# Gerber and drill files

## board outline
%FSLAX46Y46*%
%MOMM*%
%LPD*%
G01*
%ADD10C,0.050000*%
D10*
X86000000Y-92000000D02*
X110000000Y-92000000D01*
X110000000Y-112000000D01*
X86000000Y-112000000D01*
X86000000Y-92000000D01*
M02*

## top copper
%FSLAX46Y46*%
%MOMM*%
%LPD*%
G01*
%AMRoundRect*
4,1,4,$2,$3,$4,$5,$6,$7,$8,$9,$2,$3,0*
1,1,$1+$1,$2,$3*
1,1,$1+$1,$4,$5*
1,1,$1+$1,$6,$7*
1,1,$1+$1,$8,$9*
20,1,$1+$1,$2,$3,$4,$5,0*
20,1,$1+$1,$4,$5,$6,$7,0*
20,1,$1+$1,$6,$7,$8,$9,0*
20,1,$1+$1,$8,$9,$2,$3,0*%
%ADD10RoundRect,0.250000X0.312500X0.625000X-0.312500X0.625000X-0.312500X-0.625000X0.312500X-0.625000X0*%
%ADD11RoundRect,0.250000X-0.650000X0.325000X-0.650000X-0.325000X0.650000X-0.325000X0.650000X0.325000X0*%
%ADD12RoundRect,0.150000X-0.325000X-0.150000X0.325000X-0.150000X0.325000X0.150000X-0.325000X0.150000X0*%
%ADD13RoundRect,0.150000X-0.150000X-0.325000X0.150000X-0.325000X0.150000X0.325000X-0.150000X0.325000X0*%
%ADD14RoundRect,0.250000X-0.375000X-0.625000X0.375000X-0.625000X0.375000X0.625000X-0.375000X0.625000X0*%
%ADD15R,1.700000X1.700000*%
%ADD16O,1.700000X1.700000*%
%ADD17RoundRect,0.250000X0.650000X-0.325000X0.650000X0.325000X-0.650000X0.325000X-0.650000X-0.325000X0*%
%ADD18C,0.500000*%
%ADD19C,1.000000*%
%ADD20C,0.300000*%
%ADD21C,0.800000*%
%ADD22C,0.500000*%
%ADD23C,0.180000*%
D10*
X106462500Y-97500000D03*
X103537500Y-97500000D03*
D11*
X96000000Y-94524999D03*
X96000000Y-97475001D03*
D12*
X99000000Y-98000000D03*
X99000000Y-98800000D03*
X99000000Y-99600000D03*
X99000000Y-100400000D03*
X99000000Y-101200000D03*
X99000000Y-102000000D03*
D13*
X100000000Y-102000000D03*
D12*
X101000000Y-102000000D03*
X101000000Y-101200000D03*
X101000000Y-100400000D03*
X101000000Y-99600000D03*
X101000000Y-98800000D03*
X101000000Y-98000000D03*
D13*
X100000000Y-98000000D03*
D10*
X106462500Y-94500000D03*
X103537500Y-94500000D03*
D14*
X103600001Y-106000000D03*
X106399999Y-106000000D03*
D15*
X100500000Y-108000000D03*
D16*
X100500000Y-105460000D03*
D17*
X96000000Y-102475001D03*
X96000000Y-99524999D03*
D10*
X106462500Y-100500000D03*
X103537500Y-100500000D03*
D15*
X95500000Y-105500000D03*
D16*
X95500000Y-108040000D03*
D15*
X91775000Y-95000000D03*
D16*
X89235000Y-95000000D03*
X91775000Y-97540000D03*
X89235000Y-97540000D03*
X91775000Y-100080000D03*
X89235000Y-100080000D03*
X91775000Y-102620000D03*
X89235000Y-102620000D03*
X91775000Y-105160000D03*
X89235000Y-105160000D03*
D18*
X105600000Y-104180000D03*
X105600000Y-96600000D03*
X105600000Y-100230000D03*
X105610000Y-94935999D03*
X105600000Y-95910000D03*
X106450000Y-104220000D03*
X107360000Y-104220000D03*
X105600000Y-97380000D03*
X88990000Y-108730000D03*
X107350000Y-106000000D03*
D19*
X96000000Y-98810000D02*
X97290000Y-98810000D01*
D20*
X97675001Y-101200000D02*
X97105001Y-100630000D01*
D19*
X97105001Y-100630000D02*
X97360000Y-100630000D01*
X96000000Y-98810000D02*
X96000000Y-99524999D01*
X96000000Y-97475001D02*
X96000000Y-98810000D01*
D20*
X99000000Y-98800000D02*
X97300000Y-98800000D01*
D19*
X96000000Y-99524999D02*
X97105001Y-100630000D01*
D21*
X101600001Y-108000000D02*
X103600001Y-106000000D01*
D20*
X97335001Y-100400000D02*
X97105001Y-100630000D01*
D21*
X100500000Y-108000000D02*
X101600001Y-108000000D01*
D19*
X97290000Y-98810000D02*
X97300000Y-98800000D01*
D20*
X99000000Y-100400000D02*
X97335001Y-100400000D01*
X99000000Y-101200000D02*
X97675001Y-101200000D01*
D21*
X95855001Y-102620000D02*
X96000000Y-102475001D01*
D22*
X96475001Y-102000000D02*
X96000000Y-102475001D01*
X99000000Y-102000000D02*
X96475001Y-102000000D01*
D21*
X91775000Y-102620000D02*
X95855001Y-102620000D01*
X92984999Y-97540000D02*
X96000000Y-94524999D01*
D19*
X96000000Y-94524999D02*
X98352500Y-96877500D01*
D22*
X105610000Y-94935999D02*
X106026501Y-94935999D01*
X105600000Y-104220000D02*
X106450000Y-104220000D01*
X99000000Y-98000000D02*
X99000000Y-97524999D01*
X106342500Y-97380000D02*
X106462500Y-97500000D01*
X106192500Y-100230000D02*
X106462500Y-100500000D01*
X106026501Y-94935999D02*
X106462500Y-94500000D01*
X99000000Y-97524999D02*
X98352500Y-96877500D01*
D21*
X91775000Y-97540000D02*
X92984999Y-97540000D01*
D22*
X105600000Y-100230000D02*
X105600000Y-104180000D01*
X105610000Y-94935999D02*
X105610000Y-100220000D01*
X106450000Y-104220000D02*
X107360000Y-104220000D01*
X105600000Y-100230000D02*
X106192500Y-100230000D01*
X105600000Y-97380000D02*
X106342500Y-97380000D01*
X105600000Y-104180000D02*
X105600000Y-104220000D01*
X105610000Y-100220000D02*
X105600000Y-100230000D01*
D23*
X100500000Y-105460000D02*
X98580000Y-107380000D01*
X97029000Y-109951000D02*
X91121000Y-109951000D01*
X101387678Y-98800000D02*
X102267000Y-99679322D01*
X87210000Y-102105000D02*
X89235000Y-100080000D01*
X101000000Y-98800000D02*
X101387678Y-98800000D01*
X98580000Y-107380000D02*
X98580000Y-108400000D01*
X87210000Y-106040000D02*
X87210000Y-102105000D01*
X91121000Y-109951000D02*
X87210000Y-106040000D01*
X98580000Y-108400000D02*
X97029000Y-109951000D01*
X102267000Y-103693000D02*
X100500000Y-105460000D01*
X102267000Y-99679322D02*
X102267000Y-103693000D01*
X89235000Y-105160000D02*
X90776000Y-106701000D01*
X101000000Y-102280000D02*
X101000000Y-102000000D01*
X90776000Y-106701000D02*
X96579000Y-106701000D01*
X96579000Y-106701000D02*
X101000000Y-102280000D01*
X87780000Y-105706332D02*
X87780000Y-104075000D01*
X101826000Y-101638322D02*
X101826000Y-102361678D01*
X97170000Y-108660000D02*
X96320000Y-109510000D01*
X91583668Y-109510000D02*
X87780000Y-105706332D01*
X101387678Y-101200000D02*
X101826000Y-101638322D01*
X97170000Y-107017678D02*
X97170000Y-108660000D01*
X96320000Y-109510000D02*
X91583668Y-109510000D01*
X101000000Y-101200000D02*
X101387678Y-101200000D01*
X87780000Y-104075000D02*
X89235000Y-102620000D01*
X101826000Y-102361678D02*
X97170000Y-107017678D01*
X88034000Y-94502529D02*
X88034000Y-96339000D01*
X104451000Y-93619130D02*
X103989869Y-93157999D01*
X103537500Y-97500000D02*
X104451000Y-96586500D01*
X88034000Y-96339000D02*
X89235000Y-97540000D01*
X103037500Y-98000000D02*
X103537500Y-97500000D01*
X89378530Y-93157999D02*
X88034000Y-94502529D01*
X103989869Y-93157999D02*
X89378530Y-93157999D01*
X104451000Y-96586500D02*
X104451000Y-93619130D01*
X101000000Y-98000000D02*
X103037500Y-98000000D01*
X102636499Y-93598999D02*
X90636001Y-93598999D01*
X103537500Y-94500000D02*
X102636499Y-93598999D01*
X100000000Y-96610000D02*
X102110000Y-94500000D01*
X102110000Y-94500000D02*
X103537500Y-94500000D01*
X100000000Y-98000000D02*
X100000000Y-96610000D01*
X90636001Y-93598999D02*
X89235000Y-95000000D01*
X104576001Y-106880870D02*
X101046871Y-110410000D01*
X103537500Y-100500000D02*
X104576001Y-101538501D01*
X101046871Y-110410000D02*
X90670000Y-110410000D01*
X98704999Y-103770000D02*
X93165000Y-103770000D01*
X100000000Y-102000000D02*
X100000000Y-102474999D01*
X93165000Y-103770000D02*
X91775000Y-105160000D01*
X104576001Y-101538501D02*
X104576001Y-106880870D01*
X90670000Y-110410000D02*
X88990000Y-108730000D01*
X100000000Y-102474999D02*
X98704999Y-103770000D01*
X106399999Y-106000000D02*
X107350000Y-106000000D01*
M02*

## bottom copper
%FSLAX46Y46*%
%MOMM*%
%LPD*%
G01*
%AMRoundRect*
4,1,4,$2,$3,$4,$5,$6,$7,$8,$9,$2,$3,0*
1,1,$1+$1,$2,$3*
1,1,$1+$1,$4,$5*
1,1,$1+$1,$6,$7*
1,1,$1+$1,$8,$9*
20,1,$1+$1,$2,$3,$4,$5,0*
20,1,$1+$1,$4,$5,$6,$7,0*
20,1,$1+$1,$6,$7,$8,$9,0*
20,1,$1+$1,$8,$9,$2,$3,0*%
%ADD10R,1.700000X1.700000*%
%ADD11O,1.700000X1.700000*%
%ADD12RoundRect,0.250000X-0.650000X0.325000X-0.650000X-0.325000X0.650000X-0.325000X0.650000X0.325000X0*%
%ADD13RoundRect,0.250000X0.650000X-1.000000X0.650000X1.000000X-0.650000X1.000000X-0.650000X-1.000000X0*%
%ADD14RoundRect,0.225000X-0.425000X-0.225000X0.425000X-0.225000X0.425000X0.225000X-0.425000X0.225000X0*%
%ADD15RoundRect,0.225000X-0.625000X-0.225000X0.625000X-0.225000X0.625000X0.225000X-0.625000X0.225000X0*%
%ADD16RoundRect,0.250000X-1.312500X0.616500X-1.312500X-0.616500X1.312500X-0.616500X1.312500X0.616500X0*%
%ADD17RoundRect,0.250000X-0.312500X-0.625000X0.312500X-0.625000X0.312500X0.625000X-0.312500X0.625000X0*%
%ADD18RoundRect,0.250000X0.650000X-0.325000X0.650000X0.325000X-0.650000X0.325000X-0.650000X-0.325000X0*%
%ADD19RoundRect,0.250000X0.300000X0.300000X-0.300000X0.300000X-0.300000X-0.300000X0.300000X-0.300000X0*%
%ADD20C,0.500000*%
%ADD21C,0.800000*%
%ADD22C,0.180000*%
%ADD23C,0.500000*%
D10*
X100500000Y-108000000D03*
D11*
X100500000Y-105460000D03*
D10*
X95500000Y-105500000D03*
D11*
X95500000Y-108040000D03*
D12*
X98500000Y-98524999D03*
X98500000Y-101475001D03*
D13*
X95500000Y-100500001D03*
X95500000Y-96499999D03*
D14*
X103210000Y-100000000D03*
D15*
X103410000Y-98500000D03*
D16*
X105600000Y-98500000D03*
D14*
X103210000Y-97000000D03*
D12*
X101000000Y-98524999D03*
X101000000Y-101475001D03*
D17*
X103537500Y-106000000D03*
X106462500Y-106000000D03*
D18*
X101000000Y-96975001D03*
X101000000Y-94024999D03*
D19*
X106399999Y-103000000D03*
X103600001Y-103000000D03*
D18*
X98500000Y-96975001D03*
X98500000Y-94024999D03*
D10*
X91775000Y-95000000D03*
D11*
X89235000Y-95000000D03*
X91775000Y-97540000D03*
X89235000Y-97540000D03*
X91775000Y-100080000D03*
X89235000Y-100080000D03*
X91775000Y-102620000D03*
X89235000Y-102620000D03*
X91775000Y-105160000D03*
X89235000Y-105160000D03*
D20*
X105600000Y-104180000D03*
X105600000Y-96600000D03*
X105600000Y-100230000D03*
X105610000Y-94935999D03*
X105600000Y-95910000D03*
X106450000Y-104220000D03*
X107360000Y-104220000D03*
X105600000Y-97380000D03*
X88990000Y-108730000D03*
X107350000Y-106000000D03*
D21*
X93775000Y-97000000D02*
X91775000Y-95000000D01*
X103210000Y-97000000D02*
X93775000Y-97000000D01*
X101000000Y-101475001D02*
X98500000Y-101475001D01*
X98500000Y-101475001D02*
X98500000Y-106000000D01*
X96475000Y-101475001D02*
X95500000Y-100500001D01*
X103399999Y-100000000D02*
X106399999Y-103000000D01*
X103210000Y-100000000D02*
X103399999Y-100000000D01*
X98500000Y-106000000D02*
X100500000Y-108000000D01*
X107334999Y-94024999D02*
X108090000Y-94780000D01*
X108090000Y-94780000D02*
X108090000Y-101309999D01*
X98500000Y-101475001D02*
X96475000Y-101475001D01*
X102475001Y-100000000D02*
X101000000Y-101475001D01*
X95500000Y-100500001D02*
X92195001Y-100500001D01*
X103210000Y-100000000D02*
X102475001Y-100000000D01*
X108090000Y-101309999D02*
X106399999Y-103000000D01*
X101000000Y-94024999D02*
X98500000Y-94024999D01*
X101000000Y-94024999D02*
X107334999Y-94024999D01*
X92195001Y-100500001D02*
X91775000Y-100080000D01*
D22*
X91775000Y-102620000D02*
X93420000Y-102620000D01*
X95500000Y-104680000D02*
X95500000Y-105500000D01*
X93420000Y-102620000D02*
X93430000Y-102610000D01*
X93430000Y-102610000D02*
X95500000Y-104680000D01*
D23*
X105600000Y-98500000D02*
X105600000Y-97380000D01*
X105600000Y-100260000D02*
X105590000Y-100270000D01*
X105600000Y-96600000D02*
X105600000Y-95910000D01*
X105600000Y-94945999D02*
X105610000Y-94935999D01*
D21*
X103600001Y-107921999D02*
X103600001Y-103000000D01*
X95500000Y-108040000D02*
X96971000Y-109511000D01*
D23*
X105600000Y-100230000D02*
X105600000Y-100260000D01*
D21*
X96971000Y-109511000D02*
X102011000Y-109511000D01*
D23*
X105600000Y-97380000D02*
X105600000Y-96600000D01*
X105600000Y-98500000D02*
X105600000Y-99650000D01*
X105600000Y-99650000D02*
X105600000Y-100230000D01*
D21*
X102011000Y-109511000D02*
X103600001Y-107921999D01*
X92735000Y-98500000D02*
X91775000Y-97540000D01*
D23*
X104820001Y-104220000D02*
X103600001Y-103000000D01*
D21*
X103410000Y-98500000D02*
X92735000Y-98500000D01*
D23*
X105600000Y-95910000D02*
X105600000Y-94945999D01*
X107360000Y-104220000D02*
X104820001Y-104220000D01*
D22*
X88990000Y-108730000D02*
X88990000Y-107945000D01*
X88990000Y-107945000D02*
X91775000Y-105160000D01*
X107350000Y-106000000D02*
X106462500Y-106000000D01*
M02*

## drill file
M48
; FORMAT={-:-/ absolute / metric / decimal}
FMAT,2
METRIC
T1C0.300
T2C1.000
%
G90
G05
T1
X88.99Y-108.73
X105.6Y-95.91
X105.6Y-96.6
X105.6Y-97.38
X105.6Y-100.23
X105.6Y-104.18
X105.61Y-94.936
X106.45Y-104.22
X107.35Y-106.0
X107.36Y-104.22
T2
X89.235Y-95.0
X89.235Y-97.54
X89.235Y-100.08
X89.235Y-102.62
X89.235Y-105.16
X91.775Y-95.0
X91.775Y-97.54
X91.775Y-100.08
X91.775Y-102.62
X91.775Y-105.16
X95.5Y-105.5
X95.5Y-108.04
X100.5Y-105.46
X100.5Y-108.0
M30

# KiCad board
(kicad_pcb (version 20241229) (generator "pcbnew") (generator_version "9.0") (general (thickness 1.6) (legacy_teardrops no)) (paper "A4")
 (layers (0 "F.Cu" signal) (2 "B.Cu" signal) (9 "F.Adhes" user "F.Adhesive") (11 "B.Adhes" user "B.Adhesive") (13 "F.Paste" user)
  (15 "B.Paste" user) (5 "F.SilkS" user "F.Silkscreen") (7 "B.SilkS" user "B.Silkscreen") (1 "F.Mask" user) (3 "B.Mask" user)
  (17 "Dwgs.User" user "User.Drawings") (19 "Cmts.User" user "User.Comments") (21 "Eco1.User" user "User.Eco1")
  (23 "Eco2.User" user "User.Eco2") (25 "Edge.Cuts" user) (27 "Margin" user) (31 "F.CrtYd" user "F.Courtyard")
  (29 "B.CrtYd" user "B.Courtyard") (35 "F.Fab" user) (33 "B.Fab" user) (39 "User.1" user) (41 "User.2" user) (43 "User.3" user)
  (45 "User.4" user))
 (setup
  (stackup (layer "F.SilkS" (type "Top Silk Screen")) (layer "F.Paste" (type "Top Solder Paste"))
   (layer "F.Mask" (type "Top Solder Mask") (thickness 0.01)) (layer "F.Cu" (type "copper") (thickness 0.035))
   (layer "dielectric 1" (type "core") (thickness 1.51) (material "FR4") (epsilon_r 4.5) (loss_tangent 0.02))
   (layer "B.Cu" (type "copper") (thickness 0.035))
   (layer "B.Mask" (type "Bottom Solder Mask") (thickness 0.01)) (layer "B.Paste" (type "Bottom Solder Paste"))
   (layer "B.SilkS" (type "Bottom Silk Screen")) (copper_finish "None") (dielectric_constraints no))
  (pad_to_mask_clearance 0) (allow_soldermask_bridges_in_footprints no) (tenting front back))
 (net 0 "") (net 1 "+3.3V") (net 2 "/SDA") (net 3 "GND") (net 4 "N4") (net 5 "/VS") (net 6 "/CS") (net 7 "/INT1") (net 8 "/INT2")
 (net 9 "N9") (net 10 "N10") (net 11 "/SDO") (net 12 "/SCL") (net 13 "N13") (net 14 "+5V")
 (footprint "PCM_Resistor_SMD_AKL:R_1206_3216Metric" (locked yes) (layer "F.Cu") (at 105 97.5 180)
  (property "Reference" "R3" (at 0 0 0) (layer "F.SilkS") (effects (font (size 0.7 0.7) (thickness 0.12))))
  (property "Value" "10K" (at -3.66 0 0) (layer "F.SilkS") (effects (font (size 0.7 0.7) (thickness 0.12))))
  (pad "1" smd roundrect (at -1.4625 0 180) (size 1.125 1.75) (layers "F.Cu" "F.Mask" "F.Paste") (roundrect_rratio 0.222222) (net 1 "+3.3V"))
  (pad "2" smd roundrect (at 1.4625 0 180) (size 1.125 1.75) (layers "F.Cu" "F.Mask" "F.Paste") (roundrect_rratio 0.222222) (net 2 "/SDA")))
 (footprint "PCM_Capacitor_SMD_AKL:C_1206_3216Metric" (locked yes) (layer "F.Cu") (at 96 96 -90)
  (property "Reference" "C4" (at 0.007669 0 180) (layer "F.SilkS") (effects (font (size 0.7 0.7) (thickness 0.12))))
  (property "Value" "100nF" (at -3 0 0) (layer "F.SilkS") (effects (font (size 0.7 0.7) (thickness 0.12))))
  (pad "1" smd roundrect (at -1.475001 0 270) (size 1.15 1.8) (layers "F.Cu" "F.Mask" "F.Paste") (roundrect_rratio 0.217391) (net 1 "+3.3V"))
  (pad "2" smd roundrect (at 1.475001 0 270) (size 1.15 1.8) (layers "F.Cu" "F.Mask" "F.Paste") (roundrect_rratio 0.217391) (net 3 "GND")))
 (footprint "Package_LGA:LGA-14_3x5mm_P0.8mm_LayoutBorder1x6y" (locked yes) (layer "F.Cu") (at 100 100)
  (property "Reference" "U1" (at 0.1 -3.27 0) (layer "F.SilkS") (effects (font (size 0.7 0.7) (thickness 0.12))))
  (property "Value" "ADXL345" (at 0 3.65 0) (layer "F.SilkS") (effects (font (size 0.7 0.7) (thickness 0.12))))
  (pad "1" smd roundrect (at -1 -2) (size 0.95 0.6) (layers "F.Cu" "F.Mask" "F.Paste") (roundrect_rratio 0.25) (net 1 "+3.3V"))
  (pad "2" smd roundrect (at -1 -1.2) (size 0.95 0.6) (layers "F.Cu" "F.Mask" "F.Paste") (roundrect_rratio 0.25) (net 3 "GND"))
  (pad "3" smd roundrect (at -1 -0.4) (size 0.95 0.6) (layers "F.Cu" "F.Mask" "F.Paste") (roundrect_rratio 0.25) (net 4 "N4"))
  (pad "4" smd roundrect (at -1 0.4) (size 0.95 0.6) (layers "F.Cu" "F.Mask" "F.Paste") (roundrect_rratio 0.25) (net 3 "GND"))
  (pad "5" smd roundrect (at -1 1.2) (size 0.95 0.6) (layers "F.Cu" "F.Mask" "F.Paste") (roundrect_rratio 0.25) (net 3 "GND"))
  (pad "6" smd roundrect (at -1 2) (size 0.95 0.6) (layers "F.Cu" "F.Mask" "F.Paste") (roundrect_rratio 0.25) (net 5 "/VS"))
  (pad "7" smd roundrect (at 0 2) (size 0.6 0.95) (layers "F.Cu" "F.Mask" "F.Paste") (roundrect_rratio 0.25) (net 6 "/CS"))
  (pad "8" smd roundrect (at 1 2) (size 0.95 0.6) (layers "F.Cu" "F.Mask" "F.Paste") (roundrect_rratio 0.25) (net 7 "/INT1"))
  (pad "9" smd roundrect (at 1 1.2) (size 0.95 0.6) (layers "F.Cu" "F.Mask" "F.Paste") (roundrect_rratio 0.25) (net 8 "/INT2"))
  (pad "10" smd roundrect (at 1 0.4) (size 0.95 0.6) (layers "F.Cu" "F.Mask" "F.Paste") (roundrect_rratio 0.25) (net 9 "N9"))
  (pad "11" smd roundrect (at 1 -0.4) (size 0.95 0.6) (layers "F.Cu" "F.Mask" "F.Paste") (roundrect_rratio 0.25) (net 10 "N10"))
  (pad "12" smd roundrect (at 1 -1.2) (size 0.95 0.6) (layers "F.Cu" "F.Mask" "F.Paste") (roundrect_rratio 0.25) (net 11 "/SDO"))
  (pad "13" smd roundrect (at 1 -2) (size 0.95 0.6) (layers "F.Cu" "F.Mask" "F.Paste") (roundrect_rratio 0.25) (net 2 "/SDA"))
  (pad "14" smd roundrect (at 0 -2) (size 0.6 0.95) (layers "F.Cu" "F.Mask" "F.Paste") (roundrect_rratio 0.25) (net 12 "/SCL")))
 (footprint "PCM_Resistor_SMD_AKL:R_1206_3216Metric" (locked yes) (layer "F.Cu") (at 105 94.5 180)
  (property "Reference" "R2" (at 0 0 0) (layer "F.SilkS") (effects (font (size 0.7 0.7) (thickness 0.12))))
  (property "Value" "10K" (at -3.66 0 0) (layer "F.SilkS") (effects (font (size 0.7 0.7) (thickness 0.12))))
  (pad "1" smd roundrect (at -1.4625 0 180) (size 1.125 1.75) (layers "F.Cu" "F.Mask" "F.Paste") (roundrect_rratio 0.222222) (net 1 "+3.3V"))
  (pad "2" smd roundrect (at 1.4625 0 180) (size 1.125 1.75) (layers "F.Cu" "F.Mask" "F.Paste") (roundrect_rratio 0.222222) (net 12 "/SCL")))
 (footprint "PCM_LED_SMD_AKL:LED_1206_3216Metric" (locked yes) (layer "F.Cu") (at 105 106)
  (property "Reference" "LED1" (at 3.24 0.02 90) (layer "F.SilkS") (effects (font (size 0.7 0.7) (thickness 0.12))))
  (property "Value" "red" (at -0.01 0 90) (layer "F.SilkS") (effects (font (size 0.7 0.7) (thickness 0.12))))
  (pad "1" smd roundrect (at -1.399999 0) (size 1.25 1.75) (layers "F.Cu" "F.Mask" "F.Paste") (roundrect_rratio 0.2) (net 3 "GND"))
  (pad "2" smd roundrect (at 1.399999 0) (size 1.25 1.75) (layers "F.Cu" "F.Mask" "F.Paste") (roundrect_rratio 0.2) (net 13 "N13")))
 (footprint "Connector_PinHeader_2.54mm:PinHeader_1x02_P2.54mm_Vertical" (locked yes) (layer "F.Cu") (at 100.5 108 180)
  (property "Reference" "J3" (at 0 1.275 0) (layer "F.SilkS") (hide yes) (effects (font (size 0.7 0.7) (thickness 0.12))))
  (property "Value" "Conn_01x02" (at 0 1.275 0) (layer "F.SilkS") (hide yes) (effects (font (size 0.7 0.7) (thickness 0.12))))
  (pad "1" thru_hole rect (at 0 0 180) (size 1.7 1.7) (drill 1) (layers "*.Cu" "*.Mask") (remove_unused_layers no) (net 3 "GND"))
  (pad "2" thru_hole oval (at 0 2.54 180) (size 1.7 1.7) (drill 1) (layers "*.Cu" "*.Mask") (remove_unused_layers no) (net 11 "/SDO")))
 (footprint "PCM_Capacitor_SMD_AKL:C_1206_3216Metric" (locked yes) (layer "F.Cu") (at 96 101 90)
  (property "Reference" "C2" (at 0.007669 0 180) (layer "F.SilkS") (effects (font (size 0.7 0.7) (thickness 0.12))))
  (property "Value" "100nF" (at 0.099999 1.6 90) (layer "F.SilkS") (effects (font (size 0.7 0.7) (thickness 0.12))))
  (pad "1" smd roundrect (at -1.475001 0 90) (size 1.15 1.8) (layers "F.Cu" "F.Mask" "F.Paste") (roundrect_rratio 0.217391) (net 5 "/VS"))
  (pad "2" smd roundrect (at 1.475001 0 90) (size 1.15 1.8) (layers "F.Cu" "F.Mask" "F.Paste") (roundrect_rratio 0.217391) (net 3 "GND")))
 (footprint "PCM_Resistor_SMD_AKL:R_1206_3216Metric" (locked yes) (layer "F.Cu") (at 105 100.5 180)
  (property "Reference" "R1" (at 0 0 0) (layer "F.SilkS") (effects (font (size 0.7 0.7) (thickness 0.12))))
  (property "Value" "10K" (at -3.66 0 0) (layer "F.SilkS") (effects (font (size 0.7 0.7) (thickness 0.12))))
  (pad "1" smd roundrect (at -1.4625 0 180) (size 1.125 1.75) (layers "F.Cu" "F.Mask" "F.Paste") (roundrect_rratio 0.222222) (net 1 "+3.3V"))
  (pad "2" smd roundrect (at 1.4625 0 180) (size 1.125 1.75) (layers "F.Cu" "F.Mask" "F.Paste") (roundrect_rratio 0.222222) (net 6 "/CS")))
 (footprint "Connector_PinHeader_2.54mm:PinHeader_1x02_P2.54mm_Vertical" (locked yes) (layer "F.Cu") (at 95.5 105.5)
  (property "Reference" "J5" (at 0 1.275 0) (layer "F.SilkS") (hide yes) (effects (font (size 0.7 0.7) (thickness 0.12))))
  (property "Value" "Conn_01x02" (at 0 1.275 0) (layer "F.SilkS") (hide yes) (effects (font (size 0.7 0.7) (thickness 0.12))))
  (pad "1" thru_hole rect (at 0 0) (size 1.7 1.7) (drill 1) (layers "*.Cu" "*.Mask") (remove_unused_layers no) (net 5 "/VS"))
  (pad "2" thru_hole oval (at 0 2.54) (size 1.7 1.7) (drill 1) (layers "*.Cu" "*.Mask") (remove_unused_layers no) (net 1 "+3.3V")))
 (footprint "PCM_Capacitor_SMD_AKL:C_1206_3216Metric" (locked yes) (layer "B.Cu") (at 98.5 100 -90)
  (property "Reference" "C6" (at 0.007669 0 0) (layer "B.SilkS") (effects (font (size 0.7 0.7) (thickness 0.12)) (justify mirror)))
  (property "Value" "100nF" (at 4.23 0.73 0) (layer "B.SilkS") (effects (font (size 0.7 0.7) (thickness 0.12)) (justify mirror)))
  (pad "1" smd roundrect (at -1.475001 0 270) (size 1.15 1.8) (layers "B.Cu" "B.Mask" "B.Paste") (roundrect_rratio 0.217391) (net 1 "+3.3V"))
  (pad "2" smd roundrect (at 1.475001 0 270) (size 1.15 1.8) (layers "B.Cu" "B.Mask" "B.Paste") (roundrect_rratio 0.217391) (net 3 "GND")))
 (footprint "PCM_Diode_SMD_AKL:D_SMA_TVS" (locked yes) (layer "B.Cu") (at 95.5 98.5 90)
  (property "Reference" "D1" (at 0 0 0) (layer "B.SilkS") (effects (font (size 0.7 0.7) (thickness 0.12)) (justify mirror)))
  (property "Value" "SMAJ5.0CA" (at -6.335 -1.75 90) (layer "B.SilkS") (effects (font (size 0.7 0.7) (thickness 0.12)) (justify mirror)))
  (pad "1" smd roundrect (at -2.000001 0 90) (size 2.5 1.8) (layers "B.Cu" "B.Mask" "B.Paste") (roundrect_rratio 0.1388888889) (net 3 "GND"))
  (pad "2" smd roundrect (at 2.000001 0 90) (size 2.5 1.8) (layers "B.Cu" "B.Mask" "B.Paste") (roundrect_rratio 0.1388888889) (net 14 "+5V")))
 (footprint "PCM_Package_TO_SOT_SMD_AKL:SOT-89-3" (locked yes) (layer "B.Cu") (at 104.86 98.5)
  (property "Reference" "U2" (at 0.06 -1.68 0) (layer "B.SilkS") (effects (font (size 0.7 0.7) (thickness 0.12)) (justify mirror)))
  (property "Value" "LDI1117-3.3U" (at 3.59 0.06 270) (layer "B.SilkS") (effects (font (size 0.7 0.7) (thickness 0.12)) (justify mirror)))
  (pad "1" smd roundrect (at -1.65 1.5) (size 1.3 0.9) (layers "B.Cu" "B.Mask" "B.Paste") (roundrect_rratio 0.25) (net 3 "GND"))
  (pad "2" smd roundrect (at -1.45 0) (size 1.7 0.9) (layers "B.Cu" "B.Mask" "B.Paste") (roundrect_rratio 0.25) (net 1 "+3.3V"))
  (pad "2" smd roundrect (at 0.74 0 270) (size 1.733 3.125) (layers "B.Cu" "B.Mask" "B.Paste") (roundrect_rratio 0.1442585113)
   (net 1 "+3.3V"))
  (pad "3" smd roundrect (at -1.65 -1.5) (size 1.3 0.9) (layers "B.Cu" "B.Mask" "B.Paste") (roundrect_rratio 0.25) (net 14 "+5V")))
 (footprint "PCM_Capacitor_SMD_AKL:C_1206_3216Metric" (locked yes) (layer "B.Cu") (at 101 100 -90)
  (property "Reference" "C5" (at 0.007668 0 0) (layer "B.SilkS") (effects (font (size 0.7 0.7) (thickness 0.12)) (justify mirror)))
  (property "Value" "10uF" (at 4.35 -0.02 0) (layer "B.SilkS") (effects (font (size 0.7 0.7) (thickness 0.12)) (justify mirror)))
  (pad "1" smd roundrect (at -1.475001 0 270) (size 1.15 1.8) (layers "B.Cu" "B.Mask" "B.Paste") (roundrect_rratio 0.217391) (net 1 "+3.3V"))
  (pad "2" smd roundrect (at 1.475001 0 270) (size 1.15 1.8) (layers "B.Cu" "B.Mask" "B.Paste") (roundrect_rratio 0.217391) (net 3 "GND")))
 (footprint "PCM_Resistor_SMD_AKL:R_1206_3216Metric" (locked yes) (layer "B.Cu") (at 105 106)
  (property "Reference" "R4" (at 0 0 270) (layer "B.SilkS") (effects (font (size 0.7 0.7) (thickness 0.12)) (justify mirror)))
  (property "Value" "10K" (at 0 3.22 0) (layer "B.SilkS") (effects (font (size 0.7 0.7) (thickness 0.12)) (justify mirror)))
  (pad "1" smd roundrect (at -1.4625 0) (size 1.125 1.75) (layers "B.Cu" "B.Mask" "B.Paste") (roundrect_rratio 0.222222) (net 1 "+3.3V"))
  (pad "2" smd roundrect (at 1.4625 0) (size 1.125 1.75) (layers "B.Cu" "B.Mask" "B.Paste") (roundrect_rratio 0.222222) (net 13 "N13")))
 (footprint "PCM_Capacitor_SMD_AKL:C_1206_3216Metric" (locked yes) (layer "B.Cu") (at 101 95.5 90)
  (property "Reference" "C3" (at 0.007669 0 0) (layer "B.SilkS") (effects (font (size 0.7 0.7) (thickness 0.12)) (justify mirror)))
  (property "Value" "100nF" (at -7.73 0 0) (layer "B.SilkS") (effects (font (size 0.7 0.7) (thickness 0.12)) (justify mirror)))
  (pad "1" smd roundrect (at -1.475001 0 90) (size 1.15 1.8) (layers "B.Cu" "B.Mask" "B.Paste") (roundrect_rratio 0.217391) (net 14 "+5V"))
  (pad "2" smd roundrect (at 1.475001 0 90) (size 1.15 1.8) (layers "B.Cu" "B.Mask" "B.Paste") (roundrect_rratio 0.217391) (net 3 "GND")))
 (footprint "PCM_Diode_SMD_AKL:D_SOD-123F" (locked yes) (layer "B.Cu") (at 105 103 180)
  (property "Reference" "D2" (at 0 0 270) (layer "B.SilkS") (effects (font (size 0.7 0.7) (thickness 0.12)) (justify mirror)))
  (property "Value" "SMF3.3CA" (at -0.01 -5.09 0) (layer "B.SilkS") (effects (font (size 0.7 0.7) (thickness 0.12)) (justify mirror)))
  (pad "1" smd roundrect (at -1.399999 0 180) (size 1.1 1.1) (layers "B.Cu" "B.Mask" "B.Paste") (roundrect_rratio 0.2272727273)
   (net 3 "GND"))
  (pad "2" smd roundrect (at 1.399999 0 180) (size 1.1 1.1) (layers "B.Cu" "B.Mask" "B.Paste") (roundrect_rratio 0.2272727273)
   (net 1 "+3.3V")))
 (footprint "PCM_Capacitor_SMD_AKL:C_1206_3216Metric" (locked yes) (layer "B.Cu") (at 98.5 95.5 90)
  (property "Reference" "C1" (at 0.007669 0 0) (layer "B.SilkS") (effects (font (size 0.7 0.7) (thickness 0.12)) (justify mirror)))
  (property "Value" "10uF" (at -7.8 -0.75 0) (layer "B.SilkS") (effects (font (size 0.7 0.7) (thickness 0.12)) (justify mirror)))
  (pad "1" smd roundrect (at -1.475001 0 90) (size 1.15 1.8) (layers "B.Cu" "B.Mask" "B.Paste") (roundrect_rratio 0.217391) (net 14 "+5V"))
  (pad "2" smd roundrect (at 1.475001 0 90) (size 1.15 1.8) (layers "B.Cu" "B.Mask" "B.Paste") (roundrect_rratio 0.217391) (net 3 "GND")))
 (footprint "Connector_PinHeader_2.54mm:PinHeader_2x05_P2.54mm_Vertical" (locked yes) (layer "B.Cu") (at 91.775 95 180)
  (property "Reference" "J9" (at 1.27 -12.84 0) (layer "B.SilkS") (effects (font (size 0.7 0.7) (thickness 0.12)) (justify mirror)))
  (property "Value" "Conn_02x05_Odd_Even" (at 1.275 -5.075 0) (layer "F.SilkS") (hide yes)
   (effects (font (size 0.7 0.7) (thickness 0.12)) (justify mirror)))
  (pad "1" thru_hole rect (at 0 0 180) (size 1.7 1.7) (drill 1) (layers "*.Cu" "*.Mask") (remove_unused_layers no) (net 14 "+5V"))
  (pad "2" thru_hole oval (at 2.54 0 180) (size 1.7 1.7) (drill 1) (layers "*.Cu" "*.Mask") (remove_unused_layers no) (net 12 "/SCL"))
  (pad "3" thru_hole oval (at 0 -2.54 180) (size 1.7 1.7) (drill 1) (layers "*.Cu" "*.Mask") (remove_unused_layers no) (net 1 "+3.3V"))
  (pad "4" thru_hole oval (at 2.54 -2.54 180) (size 1.7 1.7) (drill 1) (layers "*.Cu" "*.Mask") (remove_unused_layers no) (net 2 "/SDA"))
  (pad "5" thru_hole oval (at 0 -5.08 180) (size 1.7 1.7) (drill 1) (layers "*.Cu" "*.Mask") (remove_unused_layers no) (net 3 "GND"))
  (pad "6" thru_hole oval (at 2.54 -5.08 180) (size 1.7 1.7) (drill 1) (layers "*.Cu" "*.Mask") (remove_unused_layers no) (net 11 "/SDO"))
  (pad "7" thru_hole oval (at 0 -7.62 180) (size 1.7 1.7) (drill 1) (layers "*.Cu" "*.Mask") (remove_unused_layers no) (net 5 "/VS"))
  (pad "8" thru_hole oval (at 2.54 -7.62 180) (size 1.7 1.7) (drill 1) (layers "*.Cu" "*.Mask") (remove_unused_layers no) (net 8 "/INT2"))
  (pad "9" thru_hole oval (at 0 -10.16 180) (size 1.7 1.7) (drill 1) (layers "*.Cu" "*.Mask") (remove_unused_layers no) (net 6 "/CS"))
  (pad "10" thru_hole oval (at 2.54 -10.16 180) (size 1.7 1.7) (drill 1) (layers "*.Cu" "*.Mask") (remove_unused_layers no) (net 7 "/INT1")))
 (gr_rect (start 86 92) (end 110 112) (stroke (width 0.05) (type default)) (fill no) (locked yes) (layer "Edge.Cuts"))
 (segment (start 93.775 97) (end 91.775 95) (width 0.8) (layer "B.Cu") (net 14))
 (segment (start 103.21 97) (end 93.775 97) (width 0.8) (layer "B.Cu") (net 14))
 (segment (start 96 98.81) (end 97.29 98.81) (width 1) (layer "F.Cu") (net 3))
 (segment (start 97.675001 101.2) (end 97.105001 100.63) (width 0.3) (layer "F.Cu") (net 3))
 (segment (start 97.105001 100.63) (end 97.36 100.63) (width 1) (layer "F.Cu") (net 3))
 (segment (start 96 98.81) (end 96 99.524999) (width 1) (layer "F.Cu") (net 3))
 (segment (start 96 97.475001) (end 96 98.81) (width 1) (layer "F.Cu") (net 3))
 (segment (start 99 98.8) (end 97.3 98.8) (width 0.3) (layer "F.Cu") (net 3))
 (segment (start 96 99.524999) (end 97.105001 100.63) (width 1) (layer "F.Cu") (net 3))
 (segment (start 101.600001 108) (end 103.600001 106) (width 0.8) (layer "F.Cu") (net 3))
 (segment (start 97.335001 100.4) (end 97.105001 100.63) (width 0.3) (layer "F.Cu") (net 3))
 (segment (start 100.5 108) (end 101.600001 108) (width 0.8) (layer "F.Cu") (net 3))
 (segment (start 97.29 98.81) (end 97.3 98.8) (width 1) (layer "F.Cu") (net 3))
 (segment (start 99 100.4) (end 97.335001 100.4) (width 0.3) (layer "F.Cu") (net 3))
 (segment (start 99 101.2) (end 97.675001 101.2) (width 0.3) (layer "F.Cu") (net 3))
 (segment (start 101 101.475001) (end 98.5 101.475001) (width 0.8) (layer "B.Cu") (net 3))
 (segment (start 98.5 101.475001) (end 98.5 106) (width 0.8) (layer "B.Cu") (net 3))
 (segment (start 96.475 101.475001) (end 95.5 100.500001) (width 0.8) (layer "B.Cu") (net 3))
 (segment (start 103.399999 100) (end 106.399999 103) (width 0.8) (layer "B.Cu") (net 3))
 (segment (start 103.21 100) (end 103.399999 100) (width 0.8) (layer "B.Cu") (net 3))
 (segment (start 98.5 106) (end 100.5 108) (width 0.8) (layer "B.Cu") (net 3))
 (segment (start 107.334999 94.024999) (end 108.09 94.78) (width 0.8) (layer "B.Cu") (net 3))
 (segment (start 108.09 94.78) (end 108.09 101.309999) (width 0.8) (layer "B.Cu") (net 3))
 (segment (start 98.5 101.475001) (end 96.475 101.475001) (width 0.8) (layer "B.Cu") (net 3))
 (segment (start 102.475001 100) (end 101 101.475001) (width 0.8) (layer "B.Cu") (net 3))
 (segment (start 95.5 100.500001) (end 92.195001 100.500001) (width 0.8) (layer "B.Cu") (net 3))
 (segment (start 103.21 100) (end 102.475001 100) (width 0.8) (layer "B.Cu") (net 3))
 (segment (start 108.09 101.309999) (end 106.399999 103) (width 0.8) (layer "B.Cu") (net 3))
 (segment (start 101 94.024999) (end 98.5 94.024999) (width 0.8) (layer "B.Cu") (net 3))
 (segment (start 101 94.024999) (end 107.334999 94.024999) (width 0.8) (layer "B.Cu") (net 3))
 (segment (start 92.195001 100.500001) (end 91.775 100.08) (width 0.8) (layer "B.Cu") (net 3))
 (segment (start 95.855001 102.62) (end 96 102.475001) (width 0.8) (layer "F.Cu") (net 5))
 (segment (start 96.475001 102) (end 96 102.475001) (width 0.5) (layer "F.Cu") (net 5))
 (segment (start 99 102) (end 96.475001 102) (width 0.5) (layer "F.Cu") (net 5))
 (segment (start 91.775 102.62) (end 95.855001 102.62) (width 0.8) (layer "F.Cu") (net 5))
 (segment (start 91.775 102.62) (end 93.42 102.62) (width 0.18) (layer "B.Cu") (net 5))
 (segment (start 95.5 104.68) (end 95.5 105.5) (width 0.18) (layer "B.Cu") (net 5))
 (segment (start 93.42 102.62) (end 93.43 102.61) (width 0.18) (layer "B.Cu") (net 5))
 (segment (start 93.43 102.61) (end 95.5 104.68) (width 0.18) (layer "B.Cu") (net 5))
 (segment (start 92.984999 97.54) (end 96 94.524999) (width 0.8) (layer "F.Cu") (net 1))
 (segment (start 96 94.524999) (end 98.3525 96.8775) (width 1) (layer "F.Cu") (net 1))
 (segment (start 105.61 94.935999) (end 106.026501 94.935999) (width 0.5) (layer "F.Cu") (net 1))
 (segment (start 105.6 104.22) (end 106.45 104.22) (width 0.5) (layer "F.Cu") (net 1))
 (segment (start 99 98) (end 99 97.524999) (width 0.5) (layer "F.Cu") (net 1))
 (segment (start 106.3425 97.38) (end 106.4625 97.5) (width 0.5) (layer "F.Cu") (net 1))
 (segment (start 106.1925 100.23) (end 106.4625 100.5) (width 0.5) (layer "F.Cu") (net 1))
 (segment (start 106.026501 94.935999) (end 106.4625 94.5) (width 0.5) (layer "F.Cu") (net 1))
 (segment (start 99 97.524999) (end 98.3525 96.8775) (width 0.5) (layer "F.Cu") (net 1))
 (segment (start 91.775 97.54) (end 92.984999 97.54) (width 0.8) (layer "F.Cu") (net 1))
 (segment (start 105.6 100.23) (end 105.6 104.18) (width 0.5) (layer "F.Cu") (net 1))
 (segment (start 105.61 94.935999) (end 105.61 100.22) (width 0.5) (layer "F.Cu") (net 1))
 (segment (start 106.45 104.22) (end 107.36 104.22) (width 0.5) (layer "F.Cu") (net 1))
 (segment (start 105.6 100.23) (end 106.1925 100.23) (width 0.5) (layer "F.Cu") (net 1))
 (segment (start 105.6 97.38) (end 106.3425 97.38) (width 0.5) (layer "F.Cu") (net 1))
 (segment (start 105.6 104.18) (end 105.6 104.22) (width 0.5) (layer "F.Cu") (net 1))
 (segment (start 105.61 100.22) (end 105.6 100.23) (width 0.5) (layer "F.Cu") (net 1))
 (via (at 105.6 104.18) (size 0.5) (drill 0.3) (layers "F.Cu" "B.Cu") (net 1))
 (via (at 105.6 96.6) (size 0.5) (drill 0.3) (layers "F.Cu" "B.Cu") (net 1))
 (via (at 105.6 100.23) (size 0.5) (drill 0.3) (layers "F.Cu" "B.Cu") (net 1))
 (via (at 105.61 94.935999) (size 0.5) (drill 0.3) (layers "F.Cu" "B.Cu") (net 1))
 (via (at 105.6 95.91) (size 0.5) (drill 0.3) (layers "F.Cu" "B.Cu") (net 1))
 (via (at 106.45 104.22) (size 0.5) (drill 0.3) (layers "F.Cu" "B.Cu") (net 1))
 (via (at 107.36 104.22) (size 0.5) (drill 0.3) (layers "F.Cu" "B.Cu") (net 1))
 (via (at 105.6 97.38) (size 0.5) (drill 0.3) (layers "F.Cu" "B.Cu") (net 1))
 (segment (start 105.6 98.5) (end 105.6 97.38) (width 0.5) (layer "B.Cu") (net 1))
 (segment (start 105.6 100.26) (end 105.59 100.27) (width 0.5) (layer "B.Cu") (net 1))
 (segment (start 105.6 96.6) (end 105.6 95.91) (width 0.5) (layer "B.Cu") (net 1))
 (segment (start 105.6 94.945999) (end 105.61 94.935999) (width 0.5) (layer "B.Cu") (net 1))
 (segment (start 103.600001 107.921999) (end 103.600001 103) (width 0.8) (layer "B.Cu") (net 1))
 (segment (start 95.5 108.04) (end 96.971 109.511) (width 0.8) (layer "B.Cu") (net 1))
 (segment (start 105.6 100.23) (end 105.6 100.26) (width 0.5) (layer "B.Cu") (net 1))
 (segment (start 96.971 109.511) (end 102.011 109.511) (width 0.8) (layer "B.Cu") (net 1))
 (segment (start 105.6 97.38) (end 105.6 96.6) (width 0.5) (layer "B.Cu") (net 1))
 (segment (start 105.6 98.5) (end 105.6 99.65) (width 0.5) (layer "B.Cu") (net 1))
 (segment (start 105.6 99.65) (end 105.6 100.23) (width 0.5) (layer "B.Cu") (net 1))
 (segment (start 102.011 109.511) (end 103.600001 107.921999) (width 0.8) (layer "B.Cu") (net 1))
 (segment (start 92.735 98.5) (end 91.775 97.54) (width 0.8) (layer "B.Cu") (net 1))
 (segment (start 104.820001 104.22) (end 103.600001 103) (width 0.5) (layer "B.Cu") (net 1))
 (segment (start 103.41 98.5) (end 92.735 98.5) (width 0.8) (layer "B.Cu") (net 1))
 (segment (start 105.6 95.91) (end 105.6 94.945999) (width 0.5) (layer "B.Cu") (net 1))
 (segment (start 107.36 104.22) (end 104.820001 104.22) (width 0.5) (layer "B.Cu") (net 1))
 (segment (start 100.5 105.46) (end 98.58 107.38) (width 0.18) (layer "F.Cu") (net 11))
 (segment (start 97.029 109.951) (end 91.121 109.951) (width 0.18) (layer "F.Cu") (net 11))
 (segment (start 101.387678 98.8) (end 102.267 99.679322) (width 0.18) (layer "F.Cu") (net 11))
 (segment (start 87.21 102.105) (end 89.235 100.08) (width 0.18) (layer "F.Cu") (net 11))
 (segment (start 101 98.8) (end 101.387678 98.8) (width 0.18) (layer "F.Cu") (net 11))
 (segment (start 98.58 107.38) (end 98.58 108.4) (width 0.18) (layer "F.Cu") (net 11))
 (segment (start 87.21 106.04) (end 87.21 102.105) (width 0.18) (layer "F.Cu") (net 11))
 (segment (start 91.121 109.951) (end 87.21 106.04) (width 0.18) (layer "F.Cu") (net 11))
 (segment (start 98.58 108.4) (end 97.029 109.951) (width 0.18) (layer "F.Cu") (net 11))
 (segment (start 102.267 103.693) (end 100.5 105.46) (width 0.18) (layer "F.Cu") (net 11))
 (segment (start 102.267 99.679322) (end 102.267 103.693) (width 0.18) (layer "F.Cu") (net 11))
 (segment (start 89.235 105.16) (end 90.776 106.701) (width 0.18) (layer "F.Cu") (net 7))
 (segment (start 101 102.28) (end 101 102) (width 0.18) (layer "F.Cu") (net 7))
 (segment (start 90.776 106.701) (end 96.579 106.701) (width 0.18) (layer "F.Cu") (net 7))
 (segment (start 96.579 106.701) (end 101 102.28) (width 0.18) (layer "F.Cu") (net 7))
 (segment (start 87.78 105.706332) (end 87.78 104.075) (width 0.18) (layer "F.Cu") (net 8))
 (segment (start 101.826 101.638322) (end 101.826 102.361678) (width 0.18) (layer "F.Cu") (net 8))
 (segment (start 97.17 108.66) (end 96.32 109.51) (width 0.18) (layer "F.Cu") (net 8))
 (segment (start 91.583668 109.51) (end 87.78 105.706332) (width 0.18) (layer "F.Cu") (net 8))
 (segment (start 101.387678 101.2) (end 101.826 101.638322) (width 0.18) (layer "F.Cu") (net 8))
 (segment (start 97.17 107.017678) (end 97.17 108.66) (width 0.18) (layer "F.Cu") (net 8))
 (segment (start 96.32 109.51) (end 91.583668 109.51) (width 0.18) (layer "F.Cu") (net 8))
 (segment (start 101 101.2) (end 101.387678 101.2) (width 0.18) (layer "F.Cu") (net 8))
 (segment (start 87.78 104.075) (end 89.235 102.62) (width 0.18) (layer "F.Cu") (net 8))
 (segment (start 101.826 102.361678) (end 97.17 107.017678) (width 0.18) (layer "F.Cu") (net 8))
 (segment (start 88.034 94.502529) (end 88.034 96.339) (width 0.18) (layer "F.Cu") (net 2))
 (segment (start 104.451 93.61913) (end 103.989869 93.157999) (width 0.18) (layer "F.Cu") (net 2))
 (segment (start 103.5375 97.5) (end 104.451 96.5865) (width 0.18) (layer "F.Cu") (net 2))
 (segment (start 88.034 96.339) (end 89.235 97.54) (width 0.18) (layer "F.Cu") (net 2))
 (segment (start 103.0375 98) (end 103.5375 97.5) (width 0.18) (layer "F.Cu") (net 2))
 (segment (start 89.37853 93.157999) (end 88.034 94.502529) (width 0.18) (layer "F.Cu") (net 2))
 (segment (start 103.989869 93.157999) (end 89.37853 93.157999) (width 0.18) (layer "F.Cu") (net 2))
 (segment (start 104.451 96.5865) (end 104.451 93.61913) (width 0.18) (layer "F.Cu") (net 2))
 (segment (start 101 98) (end 103.0375 98) (width 0.18) (layer "F.Cu") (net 2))
 (segment (start 102.636499 93.598999) (end 90.636001 93.598999) (width 0.18) (layer "F.Cu") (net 12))
 (segment (start 103.5375 94.5) (end 102.636499 93.598999) (width 0.18) (layer "F.Cu") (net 12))
 (segment (start 100 96.61) (end 102.11 94.5) (width 0.18) (layer "F.Cu") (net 12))
 (segment (start 102.11 94.5) (end 103.5375 94.5) (width 0.18) (layer "F.Cu") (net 12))
 (segment (start 100 98) (end 100 96.61) (width 0.18) (layer "F.Cu") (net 12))
 (segment (start 90.636001 93.598999) (end 89.235 95) (width 0.18) (layer "F.Cu") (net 12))
 (segment (start 104.576001 106.88087) (end 101.046871 110.41) (width 0.18) (layer "F.Cu") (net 6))
 (segment (start 103.5375 100.5) (end 104.576001 101.538501) (width 0.18) (layer "F.Cu") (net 6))
 (segment (start 101.046871 110.41) (end 90.67 110.41) (width 0.18) (layer "F.Cu") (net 6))
 (segment (start 98.704999 103.77) (end 93.165 103.77) (width 0.18) (layer "F.Cu") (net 6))
 (segment (start 100 102) (end 100 102.474999) (width 0.18) (layer "F.Cu") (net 6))
 (segment (start 93.165 103.77) (end 91.775 105.16) (width 0.18) (layer "F.Cu") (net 6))
 (segment (start 104.576001 101.538501) (end 104.576001 106.88087) (width 0.18) (layer "F.Cu") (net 6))
 (segment (start 90.67 110.41) (end 88.99 108.73) (width 0.18) (layer "F.Cu") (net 6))
 (segment (start 100 102.474999) (end 98.704999 103.77) (width 0.18) (layer "F.Cu") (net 6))
 (via (at 88.99 108.73) (size 0.5) (drill 0.3) (layers "F.Cu" "B.Cu") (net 6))
 (segment (start 88.99 108.73) (end 88.99 107.945) (width 0.18) (layer "B.Cu") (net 6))
 (segment (start 88.99 107.945) (end 91.775 105.16) (width 0.18) (layer "B.Cu") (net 6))
 (segment (start 106.399999 106) (end 107.35 106) (width 0.18) (layer "F.Cu") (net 13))
 (via (at 107.35 106) (size 0.5) (drill 0.3) (layers "F.Cu" "B.Cu") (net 13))
 (segment (start 107.35 106) (end 106.4625 106) (width 0.18) (layer "B.Cu") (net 13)))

